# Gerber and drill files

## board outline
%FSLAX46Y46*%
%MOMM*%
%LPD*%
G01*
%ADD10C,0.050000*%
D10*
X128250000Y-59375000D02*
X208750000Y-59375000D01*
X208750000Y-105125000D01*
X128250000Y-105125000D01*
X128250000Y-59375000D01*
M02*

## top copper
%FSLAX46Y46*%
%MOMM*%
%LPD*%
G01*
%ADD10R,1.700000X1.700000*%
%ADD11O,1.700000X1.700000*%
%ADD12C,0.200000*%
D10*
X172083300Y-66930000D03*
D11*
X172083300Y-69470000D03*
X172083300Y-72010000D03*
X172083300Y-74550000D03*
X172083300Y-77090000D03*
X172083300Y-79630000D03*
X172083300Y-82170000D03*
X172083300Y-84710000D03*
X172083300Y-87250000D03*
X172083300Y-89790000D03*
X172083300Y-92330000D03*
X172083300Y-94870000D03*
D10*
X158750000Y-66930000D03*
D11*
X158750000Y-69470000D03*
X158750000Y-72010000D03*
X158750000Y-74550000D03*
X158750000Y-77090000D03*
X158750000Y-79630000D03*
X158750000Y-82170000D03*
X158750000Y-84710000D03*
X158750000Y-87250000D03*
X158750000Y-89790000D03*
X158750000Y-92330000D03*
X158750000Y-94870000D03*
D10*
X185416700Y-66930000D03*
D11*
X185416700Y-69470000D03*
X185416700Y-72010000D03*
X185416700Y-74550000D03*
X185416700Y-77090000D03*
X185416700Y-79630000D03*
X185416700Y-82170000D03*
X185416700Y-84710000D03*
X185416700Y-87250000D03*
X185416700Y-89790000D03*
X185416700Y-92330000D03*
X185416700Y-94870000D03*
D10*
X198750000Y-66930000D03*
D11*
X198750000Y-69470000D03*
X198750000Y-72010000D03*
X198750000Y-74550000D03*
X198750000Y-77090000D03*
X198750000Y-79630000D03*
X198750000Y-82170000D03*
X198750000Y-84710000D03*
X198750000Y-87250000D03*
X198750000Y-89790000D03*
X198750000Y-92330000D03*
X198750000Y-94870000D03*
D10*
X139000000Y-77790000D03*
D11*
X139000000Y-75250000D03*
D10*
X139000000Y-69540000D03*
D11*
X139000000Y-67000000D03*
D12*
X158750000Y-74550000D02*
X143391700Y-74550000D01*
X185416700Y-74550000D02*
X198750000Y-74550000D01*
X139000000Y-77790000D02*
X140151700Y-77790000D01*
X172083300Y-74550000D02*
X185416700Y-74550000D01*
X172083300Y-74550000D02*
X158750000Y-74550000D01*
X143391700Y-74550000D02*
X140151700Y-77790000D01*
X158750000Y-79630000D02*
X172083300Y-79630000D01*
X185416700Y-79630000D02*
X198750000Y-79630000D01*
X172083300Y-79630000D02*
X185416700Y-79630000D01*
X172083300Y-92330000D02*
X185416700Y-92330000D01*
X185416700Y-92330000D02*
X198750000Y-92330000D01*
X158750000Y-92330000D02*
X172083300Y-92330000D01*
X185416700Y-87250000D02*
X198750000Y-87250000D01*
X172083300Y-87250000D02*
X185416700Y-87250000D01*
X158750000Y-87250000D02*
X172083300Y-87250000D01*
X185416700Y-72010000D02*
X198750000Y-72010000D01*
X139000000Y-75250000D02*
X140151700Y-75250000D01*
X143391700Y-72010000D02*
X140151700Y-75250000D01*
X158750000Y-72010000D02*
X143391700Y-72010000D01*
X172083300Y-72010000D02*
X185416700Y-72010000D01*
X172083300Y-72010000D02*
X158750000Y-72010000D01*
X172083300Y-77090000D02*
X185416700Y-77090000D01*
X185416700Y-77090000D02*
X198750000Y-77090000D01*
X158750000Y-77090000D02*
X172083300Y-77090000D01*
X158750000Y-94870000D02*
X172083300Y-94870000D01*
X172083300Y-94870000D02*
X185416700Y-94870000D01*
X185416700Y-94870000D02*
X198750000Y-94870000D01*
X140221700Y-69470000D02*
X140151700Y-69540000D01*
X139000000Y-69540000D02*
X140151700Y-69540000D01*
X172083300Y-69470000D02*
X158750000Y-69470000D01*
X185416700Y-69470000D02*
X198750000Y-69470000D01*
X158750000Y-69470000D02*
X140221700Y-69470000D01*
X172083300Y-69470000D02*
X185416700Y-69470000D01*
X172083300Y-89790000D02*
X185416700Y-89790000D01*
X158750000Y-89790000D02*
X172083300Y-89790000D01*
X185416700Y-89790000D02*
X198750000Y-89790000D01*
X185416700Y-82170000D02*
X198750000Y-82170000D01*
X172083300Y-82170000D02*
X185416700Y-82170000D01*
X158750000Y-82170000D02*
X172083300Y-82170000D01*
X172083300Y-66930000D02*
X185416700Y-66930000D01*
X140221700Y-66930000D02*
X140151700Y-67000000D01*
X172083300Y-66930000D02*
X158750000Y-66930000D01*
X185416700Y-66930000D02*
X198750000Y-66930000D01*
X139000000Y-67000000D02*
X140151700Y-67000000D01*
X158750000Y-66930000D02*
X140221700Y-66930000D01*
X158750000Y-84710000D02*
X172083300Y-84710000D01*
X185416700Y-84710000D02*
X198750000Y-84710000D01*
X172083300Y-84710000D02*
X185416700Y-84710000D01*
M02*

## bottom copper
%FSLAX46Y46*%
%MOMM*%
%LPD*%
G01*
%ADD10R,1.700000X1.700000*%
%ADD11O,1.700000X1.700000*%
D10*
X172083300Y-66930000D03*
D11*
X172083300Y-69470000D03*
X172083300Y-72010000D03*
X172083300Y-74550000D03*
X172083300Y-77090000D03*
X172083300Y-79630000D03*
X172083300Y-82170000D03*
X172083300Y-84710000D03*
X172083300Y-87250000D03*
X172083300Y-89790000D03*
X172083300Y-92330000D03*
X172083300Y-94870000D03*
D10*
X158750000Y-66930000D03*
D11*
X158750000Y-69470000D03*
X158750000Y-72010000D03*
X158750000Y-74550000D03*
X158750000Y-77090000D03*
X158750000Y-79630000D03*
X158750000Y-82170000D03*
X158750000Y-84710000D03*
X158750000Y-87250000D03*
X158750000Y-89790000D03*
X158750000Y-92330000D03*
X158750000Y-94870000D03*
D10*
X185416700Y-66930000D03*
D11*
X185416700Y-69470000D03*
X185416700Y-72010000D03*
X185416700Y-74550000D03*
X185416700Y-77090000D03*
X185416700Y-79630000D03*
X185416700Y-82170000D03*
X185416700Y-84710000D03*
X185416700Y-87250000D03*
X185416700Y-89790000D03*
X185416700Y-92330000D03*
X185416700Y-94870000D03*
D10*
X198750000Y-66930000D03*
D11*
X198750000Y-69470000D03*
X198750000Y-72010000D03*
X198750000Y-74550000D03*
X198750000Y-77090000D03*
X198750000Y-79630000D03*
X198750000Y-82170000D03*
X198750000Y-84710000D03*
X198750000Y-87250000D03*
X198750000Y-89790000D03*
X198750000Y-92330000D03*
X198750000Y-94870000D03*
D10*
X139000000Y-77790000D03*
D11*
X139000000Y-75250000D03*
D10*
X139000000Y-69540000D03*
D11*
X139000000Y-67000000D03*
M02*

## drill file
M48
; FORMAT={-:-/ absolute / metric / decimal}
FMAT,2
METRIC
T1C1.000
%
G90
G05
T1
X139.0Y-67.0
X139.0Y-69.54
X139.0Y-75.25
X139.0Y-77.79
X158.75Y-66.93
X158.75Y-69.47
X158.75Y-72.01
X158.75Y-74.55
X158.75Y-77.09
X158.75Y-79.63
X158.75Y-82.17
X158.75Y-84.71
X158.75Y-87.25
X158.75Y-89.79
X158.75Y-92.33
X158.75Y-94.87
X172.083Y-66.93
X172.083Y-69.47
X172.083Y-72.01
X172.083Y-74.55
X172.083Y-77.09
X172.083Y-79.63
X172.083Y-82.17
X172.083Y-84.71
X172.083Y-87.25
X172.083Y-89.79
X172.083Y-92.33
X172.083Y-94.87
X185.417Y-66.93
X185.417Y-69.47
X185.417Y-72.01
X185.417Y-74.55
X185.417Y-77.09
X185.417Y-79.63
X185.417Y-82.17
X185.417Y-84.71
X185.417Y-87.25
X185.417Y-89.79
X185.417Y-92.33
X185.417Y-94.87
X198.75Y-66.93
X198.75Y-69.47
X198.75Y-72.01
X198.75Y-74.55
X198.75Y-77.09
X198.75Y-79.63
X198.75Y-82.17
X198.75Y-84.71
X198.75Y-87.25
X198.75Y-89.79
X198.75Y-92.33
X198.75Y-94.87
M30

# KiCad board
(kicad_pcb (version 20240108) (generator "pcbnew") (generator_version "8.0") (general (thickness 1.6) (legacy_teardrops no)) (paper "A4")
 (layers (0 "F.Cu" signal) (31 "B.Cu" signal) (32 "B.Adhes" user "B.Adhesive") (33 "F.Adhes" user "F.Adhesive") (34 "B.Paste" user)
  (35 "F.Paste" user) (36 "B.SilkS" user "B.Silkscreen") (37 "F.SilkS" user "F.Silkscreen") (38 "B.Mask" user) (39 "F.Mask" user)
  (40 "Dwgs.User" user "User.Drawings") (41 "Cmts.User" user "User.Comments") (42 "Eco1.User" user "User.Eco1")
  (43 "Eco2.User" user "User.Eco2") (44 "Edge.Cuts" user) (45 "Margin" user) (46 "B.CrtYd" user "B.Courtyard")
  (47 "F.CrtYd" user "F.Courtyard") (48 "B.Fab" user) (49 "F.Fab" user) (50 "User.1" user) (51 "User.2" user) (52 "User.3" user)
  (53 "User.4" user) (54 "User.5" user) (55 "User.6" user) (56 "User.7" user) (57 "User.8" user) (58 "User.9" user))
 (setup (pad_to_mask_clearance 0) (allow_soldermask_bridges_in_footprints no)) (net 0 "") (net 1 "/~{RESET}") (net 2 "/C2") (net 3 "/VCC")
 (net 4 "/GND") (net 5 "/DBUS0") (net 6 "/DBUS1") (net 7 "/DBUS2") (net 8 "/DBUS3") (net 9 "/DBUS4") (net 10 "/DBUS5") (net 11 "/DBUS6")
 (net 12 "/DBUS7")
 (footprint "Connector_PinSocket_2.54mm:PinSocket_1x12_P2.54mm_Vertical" (layer "F.Cu") (at 172.0833 66.93)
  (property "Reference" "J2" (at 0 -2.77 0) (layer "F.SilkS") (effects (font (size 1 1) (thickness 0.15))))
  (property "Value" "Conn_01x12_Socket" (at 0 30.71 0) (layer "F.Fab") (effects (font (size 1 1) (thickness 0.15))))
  (pad "1" thru_hole rect (at 0 0) (size 1.7 1.7) (drill 1) (layers "*.Cu" "*.Mask") (remove_unused_layers no) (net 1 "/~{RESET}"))
  (pad "2" thru_hole oval (at 0 2.54) (size 1.7 1.7) (drill 1) (layers "*.Cu" "*.Mask") (remove_unused_layers no) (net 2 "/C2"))
  (pad "3" thru_hole oval (at 0 5.08) (size 1.7 1.7) (drill 1) (layers "*.Cu" "*.Mask") (remove_unused_layers no) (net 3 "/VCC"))
  (pad "4" thru_hole oval (at 0 7.62) (size 1.7 1.7) (drill 1) (layers "*.Cu" "*.Mask") (remove_unused_layers no) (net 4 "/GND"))
  (pad "5" thru_hole oval (at 0 10.16) (size 1.7 1.7) (drill 1) (layers "*.Cu" "*.Mask") (remove_unused_layers no) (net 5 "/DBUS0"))
  (pad "6" thru_hole oval (at 0 12.7) (size 1.7 1.7) (drill 1) (layers "*.Cu" "*.Mask") (remove_unused_layers no) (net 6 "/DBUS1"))
  (pad "7" thru_hole oval (at 0 15.24) (size 1.7 1.7) (drill 1) (layers "*.Cu" "*.Mask") (remove_unused_layers no) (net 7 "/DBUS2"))
  (pad "8" thru_hole oval (at 0 17.78) (size 1.7 1.7) (drill 1) (layers "*.Cu" "*.Mask") (remove_unused_layers no) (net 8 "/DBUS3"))
  (pad "9" thru_hole oval (at 0 20.32) (size 1.7 1.7) (drill 1) (layers "*.Cu" "*.Mask") (remove_unused_layers no) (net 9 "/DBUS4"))
  (pad "10" thru_hole oval (at 0 22.86) (size 1.7 1.7) (drill 1) (layers "*.Cu" "*.Mask") (remove_unused_layers no) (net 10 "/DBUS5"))
  (pad "11" thru_hole oval (at 0 25.4) (size 1.7 1.7) (drill 1) (layers "*.Cu" "*.Mask") (remove_unused_layers no) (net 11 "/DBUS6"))
  (pad "12" thru_hole oval (at 0 27.94) (size 1.7 1.7) (drill 1) (layers "*.Cu" "*.Mask") (remove_unused_layers no) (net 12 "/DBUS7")))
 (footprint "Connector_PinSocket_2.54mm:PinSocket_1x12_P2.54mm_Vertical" (layer "F.Cu") (at 158.75 66.93)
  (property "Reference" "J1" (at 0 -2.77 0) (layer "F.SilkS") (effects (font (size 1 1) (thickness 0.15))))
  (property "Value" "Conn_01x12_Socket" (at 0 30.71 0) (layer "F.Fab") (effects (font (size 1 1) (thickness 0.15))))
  (pad "1" thru_hole rect (at 0 0) (size 1.7 1.7) (drill 1) (layers "*.Cu" "*.Mask") (remove_unused_layers no) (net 1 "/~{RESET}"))
  (pad "2" thru_hole oval (at 0 2.54) (size 1.7 1.7) (drill 1) (layers "*.Cu" "*.Mask") (remove_unused_layers no) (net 2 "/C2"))
  (pad "3" thru_hole oval (at 0 5.08) (size 1.7 1.7) (drill 1) (layers "*.Cu" "*.Mask") (remove_unused_layers no) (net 3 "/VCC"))
  (pad "4" thru_hole oval (at 0 7.62) (size 1.7 1.7) (drill 1) (layers "*.Cu" "*.Mask") (remove_unused_layers no) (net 4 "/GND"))
  (pad "5" thru_hole oval (at 0 10.16) (size 1.7 1.7) (drill 1) (layers "*.Cu" "*.Mask") (remove_unused_layers no) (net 5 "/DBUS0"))
  (pad "6" thru_hole oval (at 0 12.7) (size 1.7 1.7) (drill 1) (layers "*.Cu" "*.Mask") (remove_unused_layers no) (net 6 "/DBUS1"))
  (pad "7" thru_hole oval (at 0 15.24) (size 1.7 1.7) (drill 1) (layers "*.Cu" "*.Mask") (remove_unused_layers no) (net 7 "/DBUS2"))
  (pad "8" thru_hole oval (at 0 17.78) (size 1.7 1.7) (drill 1) (layers "*.Cu" "*.Mask") (remove_unused_layers no) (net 8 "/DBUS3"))
  (pad "9" thru_hole oval (at 0 20.32) (size 1.7 1.7) (drill 1) (layers "*.Cu" "*.Mask") (remove_unused_layers no) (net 9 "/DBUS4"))
  (pad "10" thru_hole oval (at 0 22.86) (size 1.7 1.7) (drill 1) (layers "*.Cu" "*.Mask") (remove_unused_layers no) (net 10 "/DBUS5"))
  (pad "11" thru_hole oval (at 0 25.4) (size 1.7 1.7) (drill 1) (layers "*.Cu" "*.Mask") (remove_unused_layers no) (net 11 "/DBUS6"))
  (pad "12" thru_hole oval (at 0 27.94) (size 1.7 1.7) (drill 1) (layers "*.Cu" "*.Mask") (remove_unused_layers no) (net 12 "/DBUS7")))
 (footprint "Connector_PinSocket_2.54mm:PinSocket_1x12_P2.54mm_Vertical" (layer "F.Cu") (at 185.4167 66.93)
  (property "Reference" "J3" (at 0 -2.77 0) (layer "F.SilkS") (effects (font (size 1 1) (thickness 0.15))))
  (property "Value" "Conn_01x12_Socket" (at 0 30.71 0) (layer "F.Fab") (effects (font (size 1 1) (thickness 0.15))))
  (pad "1" thru_hole rect (at 0 0) (size 1.7 1.7) (drill 1) (layers "*.Cu" "*.Mask") (remove_unused_layers no) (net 1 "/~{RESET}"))
  (pad "2" thru_hole oval (at 0 2.54) (size 1.7 1.7) (drill 1) (layers "*.Cu" "*.Mask") (remove_unused_layers no) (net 2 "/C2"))
  (pad "3" thru_hole oval (at 0 5.08) (size 1.7 1.7) (drill 1) (layers "*.Cu" "*.Mask") (remove_unused_layers no) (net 3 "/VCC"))
  (pad "4" thru_hole oval (at 0 7.62) (size 1.7 1.7) (drill 1) (layers "*.Cu" "*.Mask") (remove_unused_layers no) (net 4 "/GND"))
  (pad "5" thru_hole oval (at 0 10.16) (size 1.7 1.7) (drill 1) (layers "*.Cu" "*.Mask") (remove_unused_layers no) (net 5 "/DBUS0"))
  (pad "6" thru_hole oval (at 0 12.7) (size 1.7 1.7) (drill 1) (layers "*.Cu" "*.Mask") (remove_unused_layers no) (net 6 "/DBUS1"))
  (pad "7" thru_hole oval (at 0 15.24) (size 1.7 1.7) (drill 1) (layers "*.Cu" "*.Mask") (remove_unused_layers no) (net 7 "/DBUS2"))
  (pad "8" thru_hole oval (at 0 17.78) (size 1.7 1.7) (drill 1) (layers "*.Cu" "*.Mask") (remove_unused_layers no) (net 8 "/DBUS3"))
  (pad "9" thru_hole oval (at 0 20.32) (size 1.7 1.7) (drill 1) (layers "*.Cu" "*.Mask") (remove_unused_layers no) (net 9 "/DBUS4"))
  (pad "10" thru_hole oval (at 0 22.86) (size 1.7 1.7) (drill 1) (layers "*.Cu" "*.Mask") (remove_unused_layers no) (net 10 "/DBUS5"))
  (pad "11" thru_hole oval (at 0 25.4) (size 1.7 1.7) (drill 1) (layers "*.Cu" "*.Mask") (remove_unused_layers no) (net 11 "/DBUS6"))
  (pad "12" thru_hole oval (at 0 27.94) (size 1.7 1.7) (drill 1) (layers "*.Cu" "*.Mask") (remove_unused_layers no) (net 12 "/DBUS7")))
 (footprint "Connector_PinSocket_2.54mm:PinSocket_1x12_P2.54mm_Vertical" (layer "F.Cu") (at 198.75 66.93)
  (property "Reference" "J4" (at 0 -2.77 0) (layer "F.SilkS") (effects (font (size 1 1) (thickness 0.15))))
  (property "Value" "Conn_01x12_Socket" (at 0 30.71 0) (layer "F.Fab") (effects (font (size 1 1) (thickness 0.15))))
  (pad "1" thru_hole rect (at 0 0) (size 1.7 1.7) (drill 1) (layers "*.Cu" "*.Mask") (remove_unused_layers no) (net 1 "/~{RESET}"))
  (pad "2" thru_hole oval (at 0 2.54) (size 1.7 1.7) (drill 1) (layers "*.Cu" "*.Mask") (remove_unused_layers no) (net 2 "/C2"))
  (pad "3" thru_hole oval (at 0 5.08) (size 1.7 1.7) (drill 1) (layers "*.Cu" "*.Mask") (remove_unused_layers no) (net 3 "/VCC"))
  (pad "4" thru_hole oval (at 0 7.62) (size 1.7 1.7) (drill 1) (layers "*.Cu" "*.Mask") (remove_unused_layers no) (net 4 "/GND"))
  (pad "5" thru_hole oval (at 0 10.16) (size 1.7 1.7) (drill 1) (layers "*.Cu" "*.Mask") (remove_unused_layers no) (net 5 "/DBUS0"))
  (pad "6" thru_hole oval (at 0 12.7) (size 1.7 1.7) (drill 1) (layers "*.Cu" "*.Mask") (remove_unused_layers no) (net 6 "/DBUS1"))
  (pad "7" thru_hole oval (at 0 15.24) (size 1.7 1.7) (drill 1) (layers "*.Cu" "*.Mask") (remove_unused_layers no) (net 7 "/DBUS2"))
  (pad "8" thru_hole oval (at 0 17.78) (size 1.7 1.7) (drill 1) (layers "*.Cu" "*.Mask") (remove_unused_layers no) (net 8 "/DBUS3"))
  (pad "9" thru_hole oval (at 0 20.32) (size 1.7 1.7) (drill 1) (layers "*.Cu" "*.Mask") (remove_unused_layers no) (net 9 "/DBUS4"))
  (pad "10" thru_hole oval (at 0 22.86) (size 1.7 1.7) (drill 1) (layers "*.Cu" "*.Mask") (remove_unused_layers no) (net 10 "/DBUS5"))
  (pad "11" thru_hole oval (at 0 25.4) (size 1.7 1.7) (drill 1) (layers "*.Cu" "*.Mask") (remove_unused_layers no) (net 11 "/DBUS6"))
  (pad "12" thru_hole oval (at 0 27.94) (size 1.7 1.7) (drill 1) (layers "*.Cu" "*.Mask") (remove_unused_layers no) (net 12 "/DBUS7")))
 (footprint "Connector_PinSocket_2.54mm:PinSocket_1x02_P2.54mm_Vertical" (layer "F.Cu") (at 139 77.79 180)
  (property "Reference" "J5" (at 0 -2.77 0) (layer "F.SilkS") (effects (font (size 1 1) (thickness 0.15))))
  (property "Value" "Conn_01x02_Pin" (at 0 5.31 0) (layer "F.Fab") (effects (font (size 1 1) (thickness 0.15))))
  (pad "1" thru_hole rect (at 0 0 180) (size 1.7 1.7) (drill 1) (layers "*.Cu" "*.Mask") (remove_unused_layers no) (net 4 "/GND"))
  (pad "2" thru_hole oval (at 0 2.54 180) (size 1.7 1.7) (drill 1) (layers "*.Cu" "*.Mask") (remove_unused_layers no) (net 3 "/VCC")))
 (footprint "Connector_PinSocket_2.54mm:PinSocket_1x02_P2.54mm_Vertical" (layer "F.Cu") (at 139 69.54 180)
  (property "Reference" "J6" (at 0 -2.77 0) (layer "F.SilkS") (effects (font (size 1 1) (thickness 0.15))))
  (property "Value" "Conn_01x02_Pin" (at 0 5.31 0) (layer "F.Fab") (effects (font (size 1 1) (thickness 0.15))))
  (pad "1" thru_hole rect (at 0 0 180) (size 1.7 1.7) (drill 1) (layers "*.Cu" "*.Mask") (remove_unused_layers no) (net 2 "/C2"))
  (pad "2" thru_hole oval (at 0 2.54 180) (size 1.7 1.7) (drill 1) (layers "*.Cu" "*.Mask") (remove_unused_layers no) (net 1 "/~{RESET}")))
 (gr_rect (start 128.25 59.375) (end 208.75 105.125) (stroke (width 0.05) (type default)) (fill none) (layer "Edge.Cuts"))
 (segment (start 158.75 74.55) (end 143.3917 74.55) (width 0.2) (layer "F.Cu") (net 4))
 (segment (start 185.4167 74.55) (end 198.75 74.55) (width 0.2) (layer "F.Cu") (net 4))
 (segment (start 139 77.79) (end 140.1517 77.79) (width 0.2) (layer "F.Cu") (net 4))
 (segment (start 172.0833 74.55) (end 185.4167 74.55) (width 0.2) (layer "F.Cu") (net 4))
 (segment (start 172.0833 74.55) (end 158.75 74.55) (width 0.2) (layer "F.Cu") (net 4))
 (segment (start 143.3917 74.55) (end 140.1517 77.79) (width 0.2) (layer "F.Cu") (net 4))
 (segment (start 158.75 79.63) (end 172.0833 79.63) (width 0.2) (layer "F.Cu") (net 6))
 (segment (start 185.4167 79.63) (end 198.75 79.63) (width 0.2) (layer "F.Cu") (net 6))
 (segment (start 172.0833 79.63) (end 185.4167 79.63) (width 0.2) (layer "F.Cu") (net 6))
 (segment (start 172.0833 92.33) (end 185.4167 92.33) (width 0.2) (layer "F.Cu") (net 11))
 (segment (start 185.4167 92.33) (end 198.75 92.33) (width 0.2) (layer "F.Cu") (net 11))
 (segment (start 158.75 92.33) (end 172.0833 92.33) (width 0.2) (layer "F.Cu") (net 11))
 (segment (start 185.4167 87.25) (end 198.75 87.25) (width 0.2) (layer "F.Cu") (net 9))
 (segment (start 172.0833 87.25) (end 185.4167 87.25) (width 0.2) (layer "F.Cu") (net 9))
 (segment (start 158.75 87.25) (end 172.0833 87.25) (width 0.2) (layer "F.Cu") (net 9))
 (segment (start 185.4167 72.01) (end 198.75 72.01) (width 0.2) (layer "F.Cu") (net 3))
 (segment (start 139 75.25) (end 140.1517 75.25) (width 0.2) (layer "F.Cu") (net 3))
 (segment (start 143.3917 72.01) (end 140.1517 75.25) (width 0.2) (layer "F.Cu") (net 3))
 (segment (start 158.75 72.01) (end 143.3917 72.01) (width 0.2) (layer "F.Cu") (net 3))
 (segment (start 172.0833 72.01) (end 185.4167 72.01) (width 0.2) (layer "F.Cu") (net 3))
 (segment (start 172.0833 72.01) (end 158.75 72.01) (width 0.2) (layer "F.Cu") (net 3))
 (segment (start 172.0833 77.09) (end 185.4167 77.09) (width 0.2) (layer "F.Cu") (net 5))
 (segment (start 185.4167 77.09) (end 198.75 77.09) (width 0.2) (layer "F.Cu") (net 5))
 (segment (start 158.75 77.09) (end 172.0833 77.09) (width 0.2) (layer "F.Cu") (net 5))
 (segment (start 158.75 94.87) (end 172.0833 94.87) (width 0.2) (layer "F.Cu") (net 12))
 (segment (start 172.0833 94.87) (end 185.4167 94.87) (width 0.2) (layer "F.Cu") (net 12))
 (segment (start 185.4167 94.87) (end 198.75 94.87) (width 0.2) (layer "F.Cu") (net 12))
 (segment (start 140.2217 69.47) (end 140.1517 69.54) (width 0.2) (layer "F.Cu") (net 2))
 (segment (start 139 69.54) (end 140.1517 69.54) (width 0.2) (layer "F.Cu") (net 2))
 (segment (start 172.0833 69.47) (end 158.75 69.47) (width 0.2) (layer "F.Cu") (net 2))
 (segment (start 185.4167 69.47) (end 198.75 69.47) (width 0.2) (layer "F.Cu") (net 2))
 (segment (start 158.75 69.47) (end 140.2217 69.47) (width 0.2) (layer "F.Cu") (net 2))
 (segment (start 172.0833 69.47) (end 185.4167 69.47) (width 0.2) (layer "F.Cu") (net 2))
 (segment (start 172.0833 89.79) (end 185.4167 89.79) (width 0.2) (layer "F.Cu") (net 10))
 (segment (start 158.75 89.79) (end 172.0833 89.79) (width 0.2) (layer "F.Cu") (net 10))
 (segment (start 185.4167 89.79) (end 198.75 89.79) (width 0.2) (layer "F.Cu") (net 10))
 (segment (start 185.4167 82.17) (end 198.75 82.17) (width 0.2) (layer "F.Cu") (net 7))
 (segment (start 172.0833 82.17) (end 185.4167 82.17) (width 0.2) (layer "F.Cu") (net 7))
 (segment (start 158.75 82.17) (end 172.0833 82.17) (width 0.2) (layer "F.Cu") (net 7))
 (segment (start 172.0833 66.93) (end 185.4167 66.93) (width 0.2) (layer "F.Cu") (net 1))
 (segment (start 140.2217 66.93) (end 140.1517 67) (width 0.2) (layer "F.Cu") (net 1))
 (segment (start 172.0833 66.93) (end 158.75 66.93) (width 0.2) (layer "F.Cu") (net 1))
 (segment (start 185.4167 66.93) (end 198.75 66.93) (width 0.2) (layer "F.Cu") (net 1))
 (segment (start 139 67) (end 140.1517 67) (width 0.2) (layer "F.Cu") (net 1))
 (segment (start 158.75 66.93) (end 140.2217 66.93) (width 0.2) (layer "F.Cu") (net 1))
 (segment (start 158.75 84.71) (end 172.0833 84.71) (width 0.2) (layer "F.Cu") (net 8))
 (segment (start 185.4167 84.71) (end 198.75 84.71) (width 0.2) (layer "F.Cu") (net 8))
 (segment (start 172.0833 84.71) (end 185.4167 84.71) (width 0.2) (layer "F.Cu") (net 8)))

